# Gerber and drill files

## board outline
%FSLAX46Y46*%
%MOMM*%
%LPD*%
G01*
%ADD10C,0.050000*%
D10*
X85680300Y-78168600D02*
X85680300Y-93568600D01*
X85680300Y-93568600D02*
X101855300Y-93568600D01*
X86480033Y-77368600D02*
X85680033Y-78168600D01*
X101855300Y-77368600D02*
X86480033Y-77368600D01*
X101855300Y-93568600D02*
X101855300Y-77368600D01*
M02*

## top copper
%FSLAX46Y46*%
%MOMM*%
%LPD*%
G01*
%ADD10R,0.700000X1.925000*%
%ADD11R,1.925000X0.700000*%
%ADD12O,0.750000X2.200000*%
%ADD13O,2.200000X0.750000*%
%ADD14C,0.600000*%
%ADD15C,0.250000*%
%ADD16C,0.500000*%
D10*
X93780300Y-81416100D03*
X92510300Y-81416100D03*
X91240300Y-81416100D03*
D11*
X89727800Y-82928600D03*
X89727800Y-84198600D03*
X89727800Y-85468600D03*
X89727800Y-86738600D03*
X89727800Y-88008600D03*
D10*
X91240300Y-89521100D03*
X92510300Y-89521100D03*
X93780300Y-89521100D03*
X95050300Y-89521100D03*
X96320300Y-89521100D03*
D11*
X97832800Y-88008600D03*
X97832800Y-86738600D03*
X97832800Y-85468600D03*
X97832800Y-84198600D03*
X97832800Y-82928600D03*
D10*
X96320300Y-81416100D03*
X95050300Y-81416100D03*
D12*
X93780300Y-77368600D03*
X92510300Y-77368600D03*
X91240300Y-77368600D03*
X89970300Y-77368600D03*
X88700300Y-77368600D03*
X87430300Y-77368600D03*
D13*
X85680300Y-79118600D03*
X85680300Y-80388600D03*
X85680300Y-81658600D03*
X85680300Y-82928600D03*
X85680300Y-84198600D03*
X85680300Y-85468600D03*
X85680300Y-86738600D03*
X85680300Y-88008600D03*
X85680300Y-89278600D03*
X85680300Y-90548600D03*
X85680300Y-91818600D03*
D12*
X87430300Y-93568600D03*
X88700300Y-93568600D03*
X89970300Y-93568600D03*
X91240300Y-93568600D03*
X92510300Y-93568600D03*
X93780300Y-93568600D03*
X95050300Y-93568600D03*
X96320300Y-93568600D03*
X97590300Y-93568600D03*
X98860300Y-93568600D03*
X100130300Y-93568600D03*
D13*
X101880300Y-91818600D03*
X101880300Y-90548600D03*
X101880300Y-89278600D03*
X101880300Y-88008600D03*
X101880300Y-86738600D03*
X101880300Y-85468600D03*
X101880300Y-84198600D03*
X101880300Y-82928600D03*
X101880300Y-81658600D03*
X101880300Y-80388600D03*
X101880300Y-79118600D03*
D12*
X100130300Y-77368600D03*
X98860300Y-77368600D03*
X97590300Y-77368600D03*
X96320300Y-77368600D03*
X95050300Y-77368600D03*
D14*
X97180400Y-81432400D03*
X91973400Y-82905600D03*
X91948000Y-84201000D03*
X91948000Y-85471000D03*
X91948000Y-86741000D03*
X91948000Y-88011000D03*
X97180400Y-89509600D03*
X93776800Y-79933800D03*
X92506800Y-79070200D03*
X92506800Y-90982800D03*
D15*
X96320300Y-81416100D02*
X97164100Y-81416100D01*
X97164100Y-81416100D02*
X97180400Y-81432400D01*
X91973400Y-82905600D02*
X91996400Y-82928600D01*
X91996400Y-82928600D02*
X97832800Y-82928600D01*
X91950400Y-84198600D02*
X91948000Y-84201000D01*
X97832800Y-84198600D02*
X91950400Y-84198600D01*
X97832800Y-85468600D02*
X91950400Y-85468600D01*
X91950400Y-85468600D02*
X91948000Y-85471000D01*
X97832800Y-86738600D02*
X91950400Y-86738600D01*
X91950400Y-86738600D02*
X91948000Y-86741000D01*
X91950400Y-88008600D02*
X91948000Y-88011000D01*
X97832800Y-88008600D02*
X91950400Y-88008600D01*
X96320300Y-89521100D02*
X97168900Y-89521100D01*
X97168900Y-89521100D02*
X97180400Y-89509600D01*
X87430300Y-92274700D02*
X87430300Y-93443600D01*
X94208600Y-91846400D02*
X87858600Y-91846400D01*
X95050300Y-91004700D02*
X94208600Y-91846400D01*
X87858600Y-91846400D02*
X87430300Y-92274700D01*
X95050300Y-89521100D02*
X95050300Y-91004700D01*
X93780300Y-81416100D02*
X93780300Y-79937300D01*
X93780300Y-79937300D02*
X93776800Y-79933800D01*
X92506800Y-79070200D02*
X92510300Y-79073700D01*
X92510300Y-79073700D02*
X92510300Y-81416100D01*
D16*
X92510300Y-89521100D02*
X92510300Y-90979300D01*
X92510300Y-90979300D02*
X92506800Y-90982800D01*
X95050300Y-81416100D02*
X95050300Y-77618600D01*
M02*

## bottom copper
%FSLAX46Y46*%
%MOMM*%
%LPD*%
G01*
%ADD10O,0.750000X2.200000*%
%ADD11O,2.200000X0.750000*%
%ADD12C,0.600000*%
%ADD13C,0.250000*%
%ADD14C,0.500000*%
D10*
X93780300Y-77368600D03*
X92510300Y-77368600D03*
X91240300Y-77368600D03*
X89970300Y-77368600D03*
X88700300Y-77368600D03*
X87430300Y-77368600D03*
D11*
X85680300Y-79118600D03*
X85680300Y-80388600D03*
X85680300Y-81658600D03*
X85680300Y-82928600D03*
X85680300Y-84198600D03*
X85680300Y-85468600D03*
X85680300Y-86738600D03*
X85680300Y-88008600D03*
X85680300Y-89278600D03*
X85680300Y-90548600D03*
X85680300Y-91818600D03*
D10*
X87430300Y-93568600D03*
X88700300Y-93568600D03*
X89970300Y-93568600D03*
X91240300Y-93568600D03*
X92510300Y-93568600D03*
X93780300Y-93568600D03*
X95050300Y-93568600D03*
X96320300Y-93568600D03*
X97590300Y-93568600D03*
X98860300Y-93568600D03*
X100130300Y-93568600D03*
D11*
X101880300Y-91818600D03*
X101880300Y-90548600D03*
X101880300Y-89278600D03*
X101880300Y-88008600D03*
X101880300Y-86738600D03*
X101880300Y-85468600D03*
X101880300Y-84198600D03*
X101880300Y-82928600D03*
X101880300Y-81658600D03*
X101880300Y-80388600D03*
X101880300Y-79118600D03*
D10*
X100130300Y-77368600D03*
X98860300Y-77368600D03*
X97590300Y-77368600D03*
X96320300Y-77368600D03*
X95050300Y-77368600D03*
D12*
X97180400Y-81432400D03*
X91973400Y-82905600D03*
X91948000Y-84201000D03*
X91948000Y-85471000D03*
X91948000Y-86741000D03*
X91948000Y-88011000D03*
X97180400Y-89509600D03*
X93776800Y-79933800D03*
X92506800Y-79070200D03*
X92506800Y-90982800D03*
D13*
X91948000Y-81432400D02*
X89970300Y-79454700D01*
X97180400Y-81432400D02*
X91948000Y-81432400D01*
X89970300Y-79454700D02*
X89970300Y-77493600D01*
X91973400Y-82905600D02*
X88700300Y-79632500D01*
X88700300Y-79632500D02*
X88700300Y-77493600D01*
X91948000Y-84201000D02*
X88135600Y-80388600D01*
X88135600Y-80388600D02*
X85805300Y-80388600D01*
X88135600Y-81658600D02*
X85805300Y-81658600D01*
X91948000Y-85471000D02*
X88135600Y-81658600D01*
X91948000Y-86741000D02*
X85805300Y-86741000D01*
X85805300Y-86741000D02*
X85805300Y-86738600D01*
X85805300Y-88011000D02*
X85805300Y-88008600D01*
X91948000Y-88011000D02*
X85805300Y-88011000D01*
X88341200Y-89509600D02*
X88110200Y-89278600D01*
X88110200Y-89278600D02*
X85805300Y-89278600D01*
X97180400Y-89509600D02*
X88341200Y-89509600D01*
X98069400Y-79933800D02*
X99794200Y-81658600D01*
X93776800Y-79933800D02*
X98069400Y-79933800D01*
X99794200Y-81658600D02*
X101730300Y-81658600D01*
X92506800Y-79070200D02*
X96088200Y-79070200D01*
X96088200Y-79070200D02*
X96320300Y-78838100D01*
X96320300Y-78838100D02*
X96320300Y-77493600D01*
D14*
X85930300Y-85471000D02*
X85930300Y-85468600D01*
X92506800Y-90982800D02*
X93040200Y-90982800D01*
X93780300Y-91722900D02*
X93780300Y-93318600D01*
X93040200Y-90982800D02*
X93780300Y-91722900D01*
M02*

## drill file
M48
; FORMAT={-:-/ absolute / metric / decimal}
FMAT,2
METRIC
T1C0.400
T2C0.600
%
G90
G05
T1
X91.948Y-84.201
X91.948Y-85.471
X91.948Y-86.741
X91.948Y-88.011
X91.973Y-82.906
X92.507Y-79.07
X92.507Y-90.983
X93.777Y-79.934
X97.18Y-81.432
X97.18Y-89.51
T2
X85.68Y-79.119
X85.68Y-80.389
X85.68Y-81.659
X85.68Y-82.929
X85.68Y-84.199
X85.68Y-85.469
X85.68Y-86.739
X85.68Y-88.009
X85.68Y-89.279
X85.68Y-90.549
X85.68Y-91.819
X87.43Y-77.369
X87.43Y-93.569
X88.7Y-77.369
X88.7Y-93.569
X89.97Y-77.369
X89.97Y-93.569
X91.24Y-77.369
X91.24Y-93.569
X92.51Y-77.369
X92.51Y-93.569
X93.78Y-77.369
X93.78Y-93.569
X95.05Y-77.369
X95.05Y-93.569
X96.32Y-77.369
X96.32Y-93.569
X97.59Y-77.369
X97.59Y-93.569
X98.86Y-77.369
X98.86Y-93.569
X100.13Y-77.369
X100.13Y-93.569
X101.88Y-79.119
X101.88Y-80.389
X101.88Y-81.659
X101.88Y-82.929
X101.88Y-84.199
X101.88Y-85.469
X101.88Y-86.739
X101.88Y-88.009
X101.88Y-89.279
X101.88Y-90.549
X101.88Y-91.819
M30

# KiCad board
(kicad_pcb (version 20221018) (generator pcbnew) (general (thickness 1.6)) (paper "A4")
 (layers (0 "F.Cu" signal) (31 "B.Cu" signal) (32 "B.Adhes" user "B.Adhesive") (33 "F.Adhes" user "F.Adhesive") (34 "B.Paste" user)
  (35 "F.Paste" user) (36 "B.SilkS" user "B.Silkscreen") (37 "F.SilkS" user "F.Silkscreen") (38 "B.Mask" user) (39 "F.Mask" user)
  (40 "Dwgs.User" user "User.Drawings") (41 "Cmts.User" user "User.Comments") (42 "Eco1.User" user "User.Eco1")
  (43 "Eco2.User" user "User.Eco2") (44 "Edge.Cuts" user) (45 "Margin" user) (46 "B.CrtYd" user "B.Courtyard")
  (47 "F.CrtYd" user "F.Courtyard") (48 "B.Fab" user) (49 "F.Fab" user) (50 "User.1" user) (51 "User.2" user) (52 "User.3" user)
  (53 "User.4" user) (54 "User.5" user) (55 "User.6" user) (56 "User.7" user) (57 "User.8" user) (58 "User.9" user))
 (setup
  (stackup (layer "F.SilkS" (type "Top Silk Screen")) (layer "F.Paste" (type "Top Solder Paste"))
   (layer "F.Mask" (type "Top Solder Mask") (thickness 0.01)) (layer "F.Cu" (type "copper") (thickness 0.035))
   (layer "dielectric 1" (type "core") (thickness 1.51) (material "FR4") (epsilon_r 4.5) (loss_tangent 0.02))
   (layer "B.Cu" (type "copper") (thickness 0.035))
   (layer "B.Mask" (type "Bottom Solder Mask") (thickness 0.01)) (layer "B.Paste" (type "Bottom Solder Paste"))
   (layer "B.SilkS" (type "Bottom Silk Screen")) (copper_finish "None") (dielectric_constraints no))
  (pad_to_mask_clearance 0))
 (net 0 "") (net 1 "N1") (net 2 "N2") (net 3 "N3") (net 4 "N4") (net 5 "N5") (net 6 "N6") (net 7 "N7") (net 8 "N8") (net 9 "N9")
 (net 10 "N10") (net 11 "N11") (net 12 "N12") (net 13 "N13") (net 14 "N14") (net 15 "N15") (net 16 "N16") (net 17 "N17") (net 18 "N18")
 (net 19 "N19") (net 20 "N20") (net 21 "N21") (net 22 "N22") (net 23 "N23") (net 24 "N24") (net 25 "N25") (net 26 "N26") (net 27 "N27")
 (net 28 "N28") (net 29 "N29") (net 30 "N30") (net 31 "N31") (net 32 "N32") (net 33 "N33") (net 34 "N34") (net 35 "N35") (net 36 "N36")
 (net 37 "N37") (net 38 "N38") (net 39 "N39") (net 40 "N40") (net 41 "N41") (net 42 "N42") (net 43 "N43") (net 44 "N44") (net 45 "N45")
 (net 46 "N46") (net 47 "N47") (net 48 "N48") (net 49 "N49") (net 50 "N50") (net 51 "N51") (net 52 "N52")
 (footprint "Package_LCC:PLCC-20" (layer "F.Cu") (at 93.7803 85.4686)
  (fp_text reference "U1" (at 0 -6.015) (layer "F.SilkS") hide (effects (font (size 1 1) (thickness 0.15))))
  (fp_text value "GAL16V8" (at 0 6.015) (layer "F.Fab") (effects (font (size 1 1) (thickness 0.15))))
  (pad "1" smd rect (at 0 -4.0525) (size 0.7 1.925) (layers "F.Cu" "F.Paste" "F.Mask") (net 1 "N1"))
  (pad "2" smd rect (at -1.27 -4.0525) (size 0.7 1.925) (layers "F.Cu" "F.Paste" "F.Mask") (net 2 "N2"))
  (pad "3" smd rect (at -2.54 -4.0525) (size 0.7 1.925) (layers "F.Cu" "F.Paste" "F.Mask") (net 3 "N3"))
  (pad "4" smd rect (at -4.0525 -2.54) (size 1.925 0.7) (layers "F.Cu" "F.Paste" "F.Mask") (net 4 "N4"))
  (pad "5" smd rect (at -4.0525 -1.27) (size 1.925 0.7) (layers "F.Cu" "F.Paste" "F.Mask") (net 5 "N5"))
  (pad "6" smd rect (at -4.0525 0) (size 1.925 0.7) (layers "F.Cu" "F.Paste" "F.Mask") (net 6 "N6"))
  (pad "7" smd rect (at -4.0525 1.27) (size 1.925 0.7) (layers "F.Cu" "F.Paste" "F.Mask") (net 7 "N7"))
  (pad "8" smd rect (at -4.0525 2.54) (size 1.925 0.7) (layers "F.Cu" "F.Paste" "F.Mask") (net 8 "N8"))
  (pad "9" smd rect (at -2.54 4.0525) (size 0.7 1.925) (layers "F.Cu" "F.Paste" "F.Mask") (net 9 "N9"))
  (pad "10" smd rect (at -1.27 4.0525) (size 0.7 1.925) (layers "F.Cu" "F.Paste" "F.Mask") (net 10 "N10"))
  (pad "11" smd rect (at 0 4.0525) (size 0.7 1.925) (layers "F.Cu" "F.Paste" "F.Mask") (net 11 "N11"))
  (pad "12" smd rect (at 1.27 4.0525) (size 0.7 1.925) (layers "F.Cu" "F.Paste" "F.Mask") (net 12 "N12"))
  (pad "13" smd rect (at 2.54 4.0525) (size 0.7 1.925) (layers "F.Cu" "F.Paste" "F.Mask") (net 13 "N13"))
  (pad "14" smd rect (at 4.0525 2.54) (size 1.925 0.7) (layers "F.Cu" "F.Paste" "F.Mask") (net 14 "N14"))
  (pad "15" smd rect (at 4.0525 1.27) (size 1.925 0.7) (layers "F.Cu" "F.Paste" "F.Mask") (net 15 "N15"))
  (pad "16" smd rect (at 4.0525 0) (size 1.925 0.7) (layers "F.Cu" "F.Paste" "F.Mask") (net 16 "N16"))
  (pad "17" smd rect (at 4.0525 -1.27) (size 1.925 0.7) (layers "F.Cu" "F.Paste" "F.Mask") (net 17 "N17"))
  (pad "18" smd rect (at 4.0525 -2.54) (size 1.925 0.7) (layers "F.Cu" "F.Paste" "F.Mask") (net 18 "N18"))
  (pad "19" smd rect (at 2.54 -4.0525) (size 0.7 1.925) (layers "F.Cu" "F.Paste" "F.Mask") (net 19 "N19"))
  (pad "20" smd rect (at 1.27 -4.0525) (size 0.7 1.925) (layers "F.Cu" "F.Paste" "F.Mask") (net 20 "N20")))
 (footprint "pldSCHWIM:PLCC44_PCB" (layer "F.Cu") (at 93.7803 85.4686)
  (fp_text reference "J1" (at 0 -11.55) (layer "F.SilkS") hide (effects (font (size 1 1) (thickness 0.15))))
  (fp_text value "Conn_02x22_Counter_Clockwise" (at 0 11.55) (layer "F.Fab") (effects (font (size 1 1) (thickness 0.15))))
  (fp_line (start -8.1 -7.3) (end -8.1 8.1) (stroke (width 0.05) (type default)) (layer "Edge.Cuts"))
  (fp_line (start -8.1 8.1) (end 8.075 8.1) (stroke (width 0.05) (type default)) (layer "Edge.Cuts"))
  (fp_line (start -7.300267 -8.1) (end -8.100267 -7.3) (stroke (width 0.05) (type default)) (layer "Edge.Cuts"))
  (fp_line (start 8.075 -8.1) (end -7.300267 -8.1) (stroke (width 0.05) (type default)) (layer "Edge.Cuts"))
  (fp_line (start 8.075 8.1) (end 8.075 -8.1) (stroke (width 0.05) (type default)) (layer "Edge.Cuts"))
  (pad "1" thru_hole oval (at 0 -8.1) (size 0.75 2.2) (drill 0.6) (layers "*.Cu" "*.Mask") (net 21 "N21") (thermal_bridge_angle 45))
  (pad "2" thru_hole oval (at -1.27 -8.1) (size 0.75 2.2) (drill 0.6) (layers "*.Cu" "*.Mask") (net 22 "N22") (thermal_bridge_angle 45))
  (pad "3" thru_hole oval (at -2.54 -8.1) (size 0.75 2.2) (drill 0.6) (layers "*.Cu" "*.Mask") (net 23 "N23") (thermal_bridge_angle 45))
  (pad "4" thru_hole oval (at -3.81 -8.1) (size 0.75 2.2) (drill 0.6) (layers "*.Cu" "*.Mask") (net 19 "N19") (thermal_bridge_angle 45))
  (pad "5" thru_hole oval (at -5.08 -8.1) (size 0.75 2.2) (drill 0.6) (layers "*.Cu" "*.Mask") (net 18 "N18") (thermal_bridge_angle 45))
  (pad "6" thru_hole oval (at -6.35 -8.1) (size 0.75 2.2) (drill 0.6) (layers "*.Cu" "*.Mask") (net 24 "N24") (thermal_bridge_angle 45))
  (pad "7" thru_hole oval (at -8.1 -6.35 90) (size 0.75 2.2) (drill 0.6) (layers "*.Cu" "*.Mask") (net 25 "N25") (thermal_bridge_angle 45))
  (pad "8" thru_hole oval (at -8.1 -5.08 90) (size 0.75 2.2) (drill 0.6) (layers "*.Cu" "*.Mask") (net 17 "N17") (thermal_bridge_angle 45))
  (pad "9" thru_hole oval (at -8.1 -3.81 90) (size 0.75 2.2) (drill 0.6) (layers "*.Cu" "*.Mask") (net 16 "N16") (thermal_bridge_angle 45))
  (pad "10" thru_hole oval (at -8.1 -2.54 90) (size 0.75 2.2) (drill 0.6) (layers "*.Cu" "*.Mask") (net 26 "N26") (thermal_bridge_angle 45))
  (pad "11" thru_hole oval (at -8.1 -1.27 90) (size 0.75 2.2) (drill 0.6) (layers "*.Cu" "*.Mask") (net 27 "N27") (thermal_bridge_angle 45))
  (pad "12" thru_hole oval (at -8.1 0 90) (size 0.75 2.2) (drill 0.6) (layers "*.Cu" "*.Mask") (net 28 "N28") (thermal_bridge_angle 45))
  (pad "13" thru_hole oval (at -8.1 1.27 90) (size 0.75 2.2) (drill 0.6) (layers "*.Cu" "*.Mask") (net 15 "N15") (thermal_bridge_angle 45))
  (pad "14" thru_hole oval (at -8.1 2.54 90) (size 0.75 2.2) (drill 0.6) (layers "*.Cu" "*.Mask") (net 14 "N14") (thermal_bridge_angle 45))
  (pad "15" thru_hole oval (at -8.1 3.81 90) (size 0.75 2.2) (drill 0.6) (layers "*.Cu" "*.Mask") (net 13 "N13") (thermal_bridge_angle 45))
  (pad "16" thru_hole oval (at -8.1 5.08 90) (size 0.75 2.2) (drill 0.6) (layers "*.Cu" "*.Mask") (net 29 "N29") (thermal_bridge_angle 45))
  (pad "17" thru_hole oval (at -8.1 6.35 90) (size 0.75 2.2) (drill 0.6) (layers "*.Cu" "*.Mask") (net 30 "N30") (thermal_bridge_angle 45))
  (pad "18" thru_hole oval (at -6.35 8.1) (size 0.75 2.2) (drill 0.6) (layers "*.Cu" "*.Mask") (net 12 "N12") (thermal_bridge_angle 45))
  (pad "19" thru_hole oval (at -5.08 8.1) (size 0.75 2.2) (drill 0.6) (layers "*.Cu" "*.Mask") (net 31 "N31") (thermal_bridge_angle 45))
  (pad "20" thru_hole oval (at -3.81 8.1) (size 0.75 2.2) (drill 0.6) (layers "*.Cu" "*.Mask") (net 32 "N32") (thermal_bridge_angle 45))
  (pad "21" thru_hole oval (at -2.54 8.1) (size 0.75 2.2) (drill 0.6) (layers "*.Cu" "*.Mask") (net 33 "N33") (thermal_bridge_angle 45))
  (pad "22" thru_hole oval (at -1.27 8.1) (size 0.75 2.2) (drill 0.6) (layers "*.Cu" "*.Mask") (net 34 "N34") (thermal_bridge_angle 45))
  (pad "23" thru_hole oval (at 0 8.1) (size 0.75 2.2) (drill 0.6) (layers "*.Cu" "*.Mask") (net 10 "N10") (thermal_bridge_angle 45))
  (pad "24" thru_hole oval (at 1.27 8.1) (size 0.75 2.2) (drill 0.6) (layers "*.Cu" "*.Mask") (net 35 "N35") (thermal_bridge_angle 45))
  (pad "25" thru_hole oval (at 2.54 8.1) (size 0.75 2.2) (drill 0.6) (layers "*.Cu" "*.Mask") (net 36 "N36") (thermal_bridge_angle 45))
  (pad "26" thru_hole oval (at 3.81 8.1) (size 0.75 2.2) (drill 0.6) (layers "*.Cu" "*.Mask") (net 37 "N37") (thermal_bridge_angle 45))
  (pad "27" thru_hole oval (at 5.08 8.1) (size 0.75 2.2) (drill 0.6) (layers "*.Cu" "*.Mask") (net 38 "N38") (thermal_bridge_angle 45))
  (pad "28" thru_hole oval (at 6.35 8.1) (size 0.75 2.2) (drill 0.6) (layers "*.Cu" "*.Mask") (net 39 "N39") (thermal_bridge_angle 45))
  (pad "29" thru_hole oval (at 8.1 6.35 90) (size 0.75 2.2) (drill 0.6) (layers "*.Cu" "*.Mask") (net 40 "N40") (thermal_bridge_angle 45))
  (pad "30" thru_hole oval (at 8.1 5.08 90) (size 0.75 2.2) (drill 0.6) (layers "*.Cu" "*.Mask") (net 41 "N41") (thermal_bridge_angle 45))
  (pad "31" thru_hole oval (at 8.1 3.81 90) (size 0.75 2.2) (drill 0.6) (layers "*.Cu" "*.Mask") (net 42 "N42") (thermal_bridge_angle 45))
  (pad "32" thru_hole oval (at 8.1 2.54 90) (size 0.75 2.2) (drill 0.6) (layers "*.Cu" "*.Mask") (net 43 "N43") (thermal_bridge_angle 45))
  (pad "33" thru_hole oval (at 8.1 1.27 90) (size 0.75 2.2) (drill 0.6) (layers "*.Cu" "*.Mask") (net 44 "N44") (thermal_bridge_angle 45))
  (pad "34" thru_hole oval (at 8.1 0 90) (size 0.75 2.2) (drill 0.6) (layers "*.Cu" "*.Mask") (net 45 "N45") (thermal_bridge_angle 45))
  (pad "35" thru_hole oval (at 8.1 -1.27 90) (size 0.75 2.2) (drill 0.6) (layers "*.Cu" "*.Mask") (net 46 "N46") (thermal_bridge_angle 45))
  (pad "36" thru_hole oval (at 8.1 -2.54 90) (size 0.75 2.2) (drill 0.6) (layers "*.Cu" "*.Mask") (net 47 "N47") (thermal_bridge_angle 45))
  (pad "37" thru_hole oval (at 8.1 -3.81 90) (size 0.75 2.2) (drill 0.6) (layers "*.Cu" "*.Mask") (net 1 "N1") (thermal_bridge_angle 45))
  (pad "38" thru_hole oval (at 8.1 -5.08 90) (size 0.75 2.2) (drill 0.6) (layers "*.Cu" "*.Mask") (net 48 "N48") (thermal_bridge_angle 45))
  (pad "39" thru_hole oval (at 8.1 -6.35 90) (size 0.75 2.2) (drill 0.6) (layers "*.Cu" "*.Mask") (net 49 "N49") (thermal_bridge_angle 45))
  (pad "40" thru_hole oval (at 6.35 -8.1) (size 0.75 2.2) (drill 0.6) (layers "*.Cu" "*.Mask") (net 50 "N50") (thermal_bridge_angle 45))
  (pad "41" thru_hole oval (at 5.08 -8.1) (size 0.75 2.2) (drill 0.6) (layers "*.Cu" "*.Mask") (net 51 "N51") (thermal_bridge_angle 45))
  (pad "42" thru_hole oval (at 3.81 -8.1) (size 0.75 2.2) (drill 0.6) (layers "*.Cu" "*.Mask") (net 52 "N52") (thermal_bridge_angle 45))
  (pad "43" thru_hole oval (at 2.54 -8.1) (size 0.75 2.2) (drill 0.6) (layers "*.Cu" "*.Mask") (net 2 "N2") (thermal_bridge_angle 45))
  (pad "44" thru_hole oval (at 1.27 -8.1) (size 0.75 2.2) (drill 0.6) (layers "*.Cu" "*.Mask") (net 20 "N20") (thermal_bridge_angle 45)))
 (segment (start 96.3203 81.4161) (end 97.1641 81.4161) (width 0.25) (layer "F.Cu") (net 19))
 (segment (start 97.1641 81.4161) (end 97.1804 81.4324) (width 0.25) (layer "F.Cu") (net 19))
 (via (at 97.1804 81.4324) (size 0.6) (drill 0.4) (layers "F.Cu" "B.Cu") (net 19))
 (segment (start 91.948 81.4324) (end 89.9703 79.4547) (width 0.25) (layer "B.Cu") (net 19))
 (segment (start 97.1804 81.4324) (end 91.948 81.4324) (width 0.25) (layer "B.Cu") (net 19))
 (segment (start 89.9703 79.4547) (end 89.9703 77.4936) (width 0.25) (layer "B.Cu") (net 19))
 (segment (start 91.9734 82.9056) (end 91.9964 82.9286) (width 0.25) (layer "F.Cu") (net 18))
 (segment (start 91.9964 82.9286) (end 97.8328 82.9286) (width 0.25) (layer "F.Cu") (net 18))
 (via (at 91.9734 82.9056) (size 0.6) (drill 0.4) (layers "F.Cu" "B.Cu") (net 18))
 (segment (start 91.9734 82.9056) (end 88.7003 79.6325) (width 0.25) (layer "B.Cu") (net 18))
 (segment (start 88.7003 79.6325) (end 88.7003 77.4936) (width 0.25) (layer "B.Cu") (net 18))
 (segment (start 91.9504 84.1986) (end 91.948 84.201) (width 0.25) (layer "F.Cu") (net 17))
 (segment (start 97.8328 84.1986) (end 91.9504 84.1986) (width 0.25) (layer "F.Cu") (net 17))
 (via (at 91.948 84.201) (size 0.6) (drill 0.4) (layers "F.Cu" "B.Cu") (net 17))
 (segment (start 91.948 84.201) (end 88.1356 80.3886) (width 0.25) (layer "B.Cu") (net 17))
 (segment (start 88.1356 80.3886) (end 85.8053 80.3886) (width 0.25) (layer "B.Cu") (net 17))
 (segment (start 97.8328 85.4686) (end 91.9504 85.4686) (width 0.25) (layer "F.Cu") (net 16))
 (segment (start 91.9504 85.4686) (end 91.948 85.471) (width 0.25) (layer "F.Cu") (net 16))
 (via (at 91.948 85.471) (size 0.6) (drill 0.4) (layers "F.Cu" "B.Cu") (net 16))
 (segment (start 88.1356 81.6586) (end 85.8053 81.6586) (width 0.25) (layer "B.Cu") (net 16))
 (segment (start 91.948 85.471) (end 88.1356 81.6586) (width 0.25) (layer "B.Cu") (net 16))
 (segment (start 97.8328 86.7386) (end 91.9504 86.7386) (width 0.25) (layer "F.Cu") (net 15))
 (segment (start 91.9504 86.7386) (end 91.948 86.741) (width 0.25) (layer "F.Cu") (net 15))
 (via (at 91.948 86.741) (size 0.6) (drill 0.4) (layers "F.Cu" "B.Cu") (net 15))
 (segment (start 91.948 86.741) (end 85.8053 86.741) (width 0.25) (layer "B.Cu") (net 15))
 (segment (start 85.8053 86.741) (end 85.8053 86.7386) (width 0.25) (layer "B.Cu") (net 15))
 (segment (start 91.9504 88.0086) (end 91.948 88.011) (width 0.25) (layer "F.Cu") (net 14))
 (segment (start 97.8328 88.0086) (end 91.9504 88.0086) (width 0.25) (layer "F.Cu") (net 14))
 (via (at 91.948 88.011) (size 0.6) (drill 0.4) (layers "F.Cu" "B.Cu") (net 14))
 (segment (start 85.8053 88.011) (end 85.8053 88.0086) (width 0.25) (layer "B.Cu") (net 14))
 (segment (start 91.948 88.011) (end 85.8053 88.011) (width 0.25) (layer "B.Cu") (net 14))
 (segment (start 96.3203 89.5211) (end 97.1689 89.5211) (width 0.25) (layer "F.Cu") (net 13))
 (segment (start 97.1689 89.5211) (end 97.1804 89.5096) (width 0.25) (layer "F.Cu") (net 13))
 (via (at 97.1804 89.5096) (size 0.6) (drill 0.4) (layers "F.Cu" "B.Cu") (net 13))
 (segment (start 88.3412 89.5096) (end 88.1102 89.2786) (width 0.25) (layer "B.Cu") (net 13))
 (segment (start 88.1102 89.2786) (end 85.8053 89.2786) (width 0.25) (layer "B.Cu") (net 13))
 (segment (start 97.1804 89.5096) (end 88.3412 89.5096) (width 0.25) (layer "B.Cu") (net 13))
 (segment (start 87.4303 92.2747) (end 87.4303 93.4436) (width 0.25) (layer "F.Cu") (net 12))
 (segment (start 94.2086 91.8464) (end 87.8586 91.8464) (width 0.25) (layer "F.Cu") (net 12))
 (segment (start 95.0503 91.0047) (end 94.2086 91.8464) (width 0.25) (layer "F.Cu") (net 12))
 (segment (start 87.8586 91.8464) (end 87.4303 92.2747) (width 0.25) (layer "F.Cu") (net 12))
 (segment (start 95.0503 89.5211) (end 95.0503 91.0047) (width 0.25) (layer "F.Cu") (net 12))
 (segment (start 93.7803 81.4161) (end 93.7803 79.9373) (width 0.25) (layer "F.Cu") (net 1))
 (segment (start 93.7803 79.9373) (end 93.7768 79.9338) (width 0.25) (layer "F.Cu") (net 1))
 (via (at 93.7768 79.9338) (size 0.6) (drill 0.4) (layers "F.Cu" "B.Cu") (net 1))
 (segment (start 98.0694 79.9338) (end 99.7942 81.6586) (width 0.25) (layer "B.Cu") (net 1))
 (segment (start 93.7768 79.9338) (end 98.0694 79.9338) (width 0.25) (layer "B.Cu") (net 1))
 (segment (start 99.7942 81.6586) (end 101.7303 81.6586) (width 0.25) (layer "B.Cu") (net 1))
 (segment (start 92.5068 79.0702) (end 92.5103 79.0737) (width 0.25) (layer "F.Cu") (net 2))
 (segment (start 92.5103 79.0737) (end 92.5103 81.4161) (width 0.25) (layer "F.Cu") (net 2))
 (via (at 92.5068 79.0702) (size 0.6) (drill 0.4) (layers "F.Cu" "B.Cu") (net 2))
 (segment (start 92.5068 79.0702) (end 96.0882 79.0702) (width 0.25) (layer "B.Cu") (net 2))
 (segment (start 96.0882 79.0702) (end 96.3203 78.8381) (width 0.25) (layer "B.Cu") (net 2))
 (segment (start 96.3203 78.8381) (end 96.3203 77.4936) (width 0.25) (layer "B.Cu") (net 2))
 (segment (start 85.9303 85.471) (end 85.9303 85.4686) (width 0.5) (layer "B.Cu") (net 28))
 (segment (start 92.5103 89.5211) (end 92.5103 90.9793) (width 0.5) (layer "F.Cu") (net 10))
 (segment (start 92.5103 90.9793) (end 92.5068 90.9828) (width 0.5) (layer "F.Cu") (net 10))
 (via (at 92.5068 90.9828) (size 0.6) (drill 0.4) (layers "F.Cu" "B.Cu") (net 10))
 (segment (start 92.5068 90.9828) (end 93.0402 90.9828) (width 0.5) (layer "B.Cu") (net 10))
 (segment (start 93.7803 91.7229) (end 93.7803 93.3186) (width 0.5) (layer "B.Cu") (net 10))
 (segment (start 93.0402 90.9828) (end 93.7803 91.7229) (width 0.5) (layer "B.Cu") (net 10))
 (segment (start 95.0503 81.4161) (end 95.0503 77.6186) (width 0.5) (layer "F.Cu") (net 20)))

